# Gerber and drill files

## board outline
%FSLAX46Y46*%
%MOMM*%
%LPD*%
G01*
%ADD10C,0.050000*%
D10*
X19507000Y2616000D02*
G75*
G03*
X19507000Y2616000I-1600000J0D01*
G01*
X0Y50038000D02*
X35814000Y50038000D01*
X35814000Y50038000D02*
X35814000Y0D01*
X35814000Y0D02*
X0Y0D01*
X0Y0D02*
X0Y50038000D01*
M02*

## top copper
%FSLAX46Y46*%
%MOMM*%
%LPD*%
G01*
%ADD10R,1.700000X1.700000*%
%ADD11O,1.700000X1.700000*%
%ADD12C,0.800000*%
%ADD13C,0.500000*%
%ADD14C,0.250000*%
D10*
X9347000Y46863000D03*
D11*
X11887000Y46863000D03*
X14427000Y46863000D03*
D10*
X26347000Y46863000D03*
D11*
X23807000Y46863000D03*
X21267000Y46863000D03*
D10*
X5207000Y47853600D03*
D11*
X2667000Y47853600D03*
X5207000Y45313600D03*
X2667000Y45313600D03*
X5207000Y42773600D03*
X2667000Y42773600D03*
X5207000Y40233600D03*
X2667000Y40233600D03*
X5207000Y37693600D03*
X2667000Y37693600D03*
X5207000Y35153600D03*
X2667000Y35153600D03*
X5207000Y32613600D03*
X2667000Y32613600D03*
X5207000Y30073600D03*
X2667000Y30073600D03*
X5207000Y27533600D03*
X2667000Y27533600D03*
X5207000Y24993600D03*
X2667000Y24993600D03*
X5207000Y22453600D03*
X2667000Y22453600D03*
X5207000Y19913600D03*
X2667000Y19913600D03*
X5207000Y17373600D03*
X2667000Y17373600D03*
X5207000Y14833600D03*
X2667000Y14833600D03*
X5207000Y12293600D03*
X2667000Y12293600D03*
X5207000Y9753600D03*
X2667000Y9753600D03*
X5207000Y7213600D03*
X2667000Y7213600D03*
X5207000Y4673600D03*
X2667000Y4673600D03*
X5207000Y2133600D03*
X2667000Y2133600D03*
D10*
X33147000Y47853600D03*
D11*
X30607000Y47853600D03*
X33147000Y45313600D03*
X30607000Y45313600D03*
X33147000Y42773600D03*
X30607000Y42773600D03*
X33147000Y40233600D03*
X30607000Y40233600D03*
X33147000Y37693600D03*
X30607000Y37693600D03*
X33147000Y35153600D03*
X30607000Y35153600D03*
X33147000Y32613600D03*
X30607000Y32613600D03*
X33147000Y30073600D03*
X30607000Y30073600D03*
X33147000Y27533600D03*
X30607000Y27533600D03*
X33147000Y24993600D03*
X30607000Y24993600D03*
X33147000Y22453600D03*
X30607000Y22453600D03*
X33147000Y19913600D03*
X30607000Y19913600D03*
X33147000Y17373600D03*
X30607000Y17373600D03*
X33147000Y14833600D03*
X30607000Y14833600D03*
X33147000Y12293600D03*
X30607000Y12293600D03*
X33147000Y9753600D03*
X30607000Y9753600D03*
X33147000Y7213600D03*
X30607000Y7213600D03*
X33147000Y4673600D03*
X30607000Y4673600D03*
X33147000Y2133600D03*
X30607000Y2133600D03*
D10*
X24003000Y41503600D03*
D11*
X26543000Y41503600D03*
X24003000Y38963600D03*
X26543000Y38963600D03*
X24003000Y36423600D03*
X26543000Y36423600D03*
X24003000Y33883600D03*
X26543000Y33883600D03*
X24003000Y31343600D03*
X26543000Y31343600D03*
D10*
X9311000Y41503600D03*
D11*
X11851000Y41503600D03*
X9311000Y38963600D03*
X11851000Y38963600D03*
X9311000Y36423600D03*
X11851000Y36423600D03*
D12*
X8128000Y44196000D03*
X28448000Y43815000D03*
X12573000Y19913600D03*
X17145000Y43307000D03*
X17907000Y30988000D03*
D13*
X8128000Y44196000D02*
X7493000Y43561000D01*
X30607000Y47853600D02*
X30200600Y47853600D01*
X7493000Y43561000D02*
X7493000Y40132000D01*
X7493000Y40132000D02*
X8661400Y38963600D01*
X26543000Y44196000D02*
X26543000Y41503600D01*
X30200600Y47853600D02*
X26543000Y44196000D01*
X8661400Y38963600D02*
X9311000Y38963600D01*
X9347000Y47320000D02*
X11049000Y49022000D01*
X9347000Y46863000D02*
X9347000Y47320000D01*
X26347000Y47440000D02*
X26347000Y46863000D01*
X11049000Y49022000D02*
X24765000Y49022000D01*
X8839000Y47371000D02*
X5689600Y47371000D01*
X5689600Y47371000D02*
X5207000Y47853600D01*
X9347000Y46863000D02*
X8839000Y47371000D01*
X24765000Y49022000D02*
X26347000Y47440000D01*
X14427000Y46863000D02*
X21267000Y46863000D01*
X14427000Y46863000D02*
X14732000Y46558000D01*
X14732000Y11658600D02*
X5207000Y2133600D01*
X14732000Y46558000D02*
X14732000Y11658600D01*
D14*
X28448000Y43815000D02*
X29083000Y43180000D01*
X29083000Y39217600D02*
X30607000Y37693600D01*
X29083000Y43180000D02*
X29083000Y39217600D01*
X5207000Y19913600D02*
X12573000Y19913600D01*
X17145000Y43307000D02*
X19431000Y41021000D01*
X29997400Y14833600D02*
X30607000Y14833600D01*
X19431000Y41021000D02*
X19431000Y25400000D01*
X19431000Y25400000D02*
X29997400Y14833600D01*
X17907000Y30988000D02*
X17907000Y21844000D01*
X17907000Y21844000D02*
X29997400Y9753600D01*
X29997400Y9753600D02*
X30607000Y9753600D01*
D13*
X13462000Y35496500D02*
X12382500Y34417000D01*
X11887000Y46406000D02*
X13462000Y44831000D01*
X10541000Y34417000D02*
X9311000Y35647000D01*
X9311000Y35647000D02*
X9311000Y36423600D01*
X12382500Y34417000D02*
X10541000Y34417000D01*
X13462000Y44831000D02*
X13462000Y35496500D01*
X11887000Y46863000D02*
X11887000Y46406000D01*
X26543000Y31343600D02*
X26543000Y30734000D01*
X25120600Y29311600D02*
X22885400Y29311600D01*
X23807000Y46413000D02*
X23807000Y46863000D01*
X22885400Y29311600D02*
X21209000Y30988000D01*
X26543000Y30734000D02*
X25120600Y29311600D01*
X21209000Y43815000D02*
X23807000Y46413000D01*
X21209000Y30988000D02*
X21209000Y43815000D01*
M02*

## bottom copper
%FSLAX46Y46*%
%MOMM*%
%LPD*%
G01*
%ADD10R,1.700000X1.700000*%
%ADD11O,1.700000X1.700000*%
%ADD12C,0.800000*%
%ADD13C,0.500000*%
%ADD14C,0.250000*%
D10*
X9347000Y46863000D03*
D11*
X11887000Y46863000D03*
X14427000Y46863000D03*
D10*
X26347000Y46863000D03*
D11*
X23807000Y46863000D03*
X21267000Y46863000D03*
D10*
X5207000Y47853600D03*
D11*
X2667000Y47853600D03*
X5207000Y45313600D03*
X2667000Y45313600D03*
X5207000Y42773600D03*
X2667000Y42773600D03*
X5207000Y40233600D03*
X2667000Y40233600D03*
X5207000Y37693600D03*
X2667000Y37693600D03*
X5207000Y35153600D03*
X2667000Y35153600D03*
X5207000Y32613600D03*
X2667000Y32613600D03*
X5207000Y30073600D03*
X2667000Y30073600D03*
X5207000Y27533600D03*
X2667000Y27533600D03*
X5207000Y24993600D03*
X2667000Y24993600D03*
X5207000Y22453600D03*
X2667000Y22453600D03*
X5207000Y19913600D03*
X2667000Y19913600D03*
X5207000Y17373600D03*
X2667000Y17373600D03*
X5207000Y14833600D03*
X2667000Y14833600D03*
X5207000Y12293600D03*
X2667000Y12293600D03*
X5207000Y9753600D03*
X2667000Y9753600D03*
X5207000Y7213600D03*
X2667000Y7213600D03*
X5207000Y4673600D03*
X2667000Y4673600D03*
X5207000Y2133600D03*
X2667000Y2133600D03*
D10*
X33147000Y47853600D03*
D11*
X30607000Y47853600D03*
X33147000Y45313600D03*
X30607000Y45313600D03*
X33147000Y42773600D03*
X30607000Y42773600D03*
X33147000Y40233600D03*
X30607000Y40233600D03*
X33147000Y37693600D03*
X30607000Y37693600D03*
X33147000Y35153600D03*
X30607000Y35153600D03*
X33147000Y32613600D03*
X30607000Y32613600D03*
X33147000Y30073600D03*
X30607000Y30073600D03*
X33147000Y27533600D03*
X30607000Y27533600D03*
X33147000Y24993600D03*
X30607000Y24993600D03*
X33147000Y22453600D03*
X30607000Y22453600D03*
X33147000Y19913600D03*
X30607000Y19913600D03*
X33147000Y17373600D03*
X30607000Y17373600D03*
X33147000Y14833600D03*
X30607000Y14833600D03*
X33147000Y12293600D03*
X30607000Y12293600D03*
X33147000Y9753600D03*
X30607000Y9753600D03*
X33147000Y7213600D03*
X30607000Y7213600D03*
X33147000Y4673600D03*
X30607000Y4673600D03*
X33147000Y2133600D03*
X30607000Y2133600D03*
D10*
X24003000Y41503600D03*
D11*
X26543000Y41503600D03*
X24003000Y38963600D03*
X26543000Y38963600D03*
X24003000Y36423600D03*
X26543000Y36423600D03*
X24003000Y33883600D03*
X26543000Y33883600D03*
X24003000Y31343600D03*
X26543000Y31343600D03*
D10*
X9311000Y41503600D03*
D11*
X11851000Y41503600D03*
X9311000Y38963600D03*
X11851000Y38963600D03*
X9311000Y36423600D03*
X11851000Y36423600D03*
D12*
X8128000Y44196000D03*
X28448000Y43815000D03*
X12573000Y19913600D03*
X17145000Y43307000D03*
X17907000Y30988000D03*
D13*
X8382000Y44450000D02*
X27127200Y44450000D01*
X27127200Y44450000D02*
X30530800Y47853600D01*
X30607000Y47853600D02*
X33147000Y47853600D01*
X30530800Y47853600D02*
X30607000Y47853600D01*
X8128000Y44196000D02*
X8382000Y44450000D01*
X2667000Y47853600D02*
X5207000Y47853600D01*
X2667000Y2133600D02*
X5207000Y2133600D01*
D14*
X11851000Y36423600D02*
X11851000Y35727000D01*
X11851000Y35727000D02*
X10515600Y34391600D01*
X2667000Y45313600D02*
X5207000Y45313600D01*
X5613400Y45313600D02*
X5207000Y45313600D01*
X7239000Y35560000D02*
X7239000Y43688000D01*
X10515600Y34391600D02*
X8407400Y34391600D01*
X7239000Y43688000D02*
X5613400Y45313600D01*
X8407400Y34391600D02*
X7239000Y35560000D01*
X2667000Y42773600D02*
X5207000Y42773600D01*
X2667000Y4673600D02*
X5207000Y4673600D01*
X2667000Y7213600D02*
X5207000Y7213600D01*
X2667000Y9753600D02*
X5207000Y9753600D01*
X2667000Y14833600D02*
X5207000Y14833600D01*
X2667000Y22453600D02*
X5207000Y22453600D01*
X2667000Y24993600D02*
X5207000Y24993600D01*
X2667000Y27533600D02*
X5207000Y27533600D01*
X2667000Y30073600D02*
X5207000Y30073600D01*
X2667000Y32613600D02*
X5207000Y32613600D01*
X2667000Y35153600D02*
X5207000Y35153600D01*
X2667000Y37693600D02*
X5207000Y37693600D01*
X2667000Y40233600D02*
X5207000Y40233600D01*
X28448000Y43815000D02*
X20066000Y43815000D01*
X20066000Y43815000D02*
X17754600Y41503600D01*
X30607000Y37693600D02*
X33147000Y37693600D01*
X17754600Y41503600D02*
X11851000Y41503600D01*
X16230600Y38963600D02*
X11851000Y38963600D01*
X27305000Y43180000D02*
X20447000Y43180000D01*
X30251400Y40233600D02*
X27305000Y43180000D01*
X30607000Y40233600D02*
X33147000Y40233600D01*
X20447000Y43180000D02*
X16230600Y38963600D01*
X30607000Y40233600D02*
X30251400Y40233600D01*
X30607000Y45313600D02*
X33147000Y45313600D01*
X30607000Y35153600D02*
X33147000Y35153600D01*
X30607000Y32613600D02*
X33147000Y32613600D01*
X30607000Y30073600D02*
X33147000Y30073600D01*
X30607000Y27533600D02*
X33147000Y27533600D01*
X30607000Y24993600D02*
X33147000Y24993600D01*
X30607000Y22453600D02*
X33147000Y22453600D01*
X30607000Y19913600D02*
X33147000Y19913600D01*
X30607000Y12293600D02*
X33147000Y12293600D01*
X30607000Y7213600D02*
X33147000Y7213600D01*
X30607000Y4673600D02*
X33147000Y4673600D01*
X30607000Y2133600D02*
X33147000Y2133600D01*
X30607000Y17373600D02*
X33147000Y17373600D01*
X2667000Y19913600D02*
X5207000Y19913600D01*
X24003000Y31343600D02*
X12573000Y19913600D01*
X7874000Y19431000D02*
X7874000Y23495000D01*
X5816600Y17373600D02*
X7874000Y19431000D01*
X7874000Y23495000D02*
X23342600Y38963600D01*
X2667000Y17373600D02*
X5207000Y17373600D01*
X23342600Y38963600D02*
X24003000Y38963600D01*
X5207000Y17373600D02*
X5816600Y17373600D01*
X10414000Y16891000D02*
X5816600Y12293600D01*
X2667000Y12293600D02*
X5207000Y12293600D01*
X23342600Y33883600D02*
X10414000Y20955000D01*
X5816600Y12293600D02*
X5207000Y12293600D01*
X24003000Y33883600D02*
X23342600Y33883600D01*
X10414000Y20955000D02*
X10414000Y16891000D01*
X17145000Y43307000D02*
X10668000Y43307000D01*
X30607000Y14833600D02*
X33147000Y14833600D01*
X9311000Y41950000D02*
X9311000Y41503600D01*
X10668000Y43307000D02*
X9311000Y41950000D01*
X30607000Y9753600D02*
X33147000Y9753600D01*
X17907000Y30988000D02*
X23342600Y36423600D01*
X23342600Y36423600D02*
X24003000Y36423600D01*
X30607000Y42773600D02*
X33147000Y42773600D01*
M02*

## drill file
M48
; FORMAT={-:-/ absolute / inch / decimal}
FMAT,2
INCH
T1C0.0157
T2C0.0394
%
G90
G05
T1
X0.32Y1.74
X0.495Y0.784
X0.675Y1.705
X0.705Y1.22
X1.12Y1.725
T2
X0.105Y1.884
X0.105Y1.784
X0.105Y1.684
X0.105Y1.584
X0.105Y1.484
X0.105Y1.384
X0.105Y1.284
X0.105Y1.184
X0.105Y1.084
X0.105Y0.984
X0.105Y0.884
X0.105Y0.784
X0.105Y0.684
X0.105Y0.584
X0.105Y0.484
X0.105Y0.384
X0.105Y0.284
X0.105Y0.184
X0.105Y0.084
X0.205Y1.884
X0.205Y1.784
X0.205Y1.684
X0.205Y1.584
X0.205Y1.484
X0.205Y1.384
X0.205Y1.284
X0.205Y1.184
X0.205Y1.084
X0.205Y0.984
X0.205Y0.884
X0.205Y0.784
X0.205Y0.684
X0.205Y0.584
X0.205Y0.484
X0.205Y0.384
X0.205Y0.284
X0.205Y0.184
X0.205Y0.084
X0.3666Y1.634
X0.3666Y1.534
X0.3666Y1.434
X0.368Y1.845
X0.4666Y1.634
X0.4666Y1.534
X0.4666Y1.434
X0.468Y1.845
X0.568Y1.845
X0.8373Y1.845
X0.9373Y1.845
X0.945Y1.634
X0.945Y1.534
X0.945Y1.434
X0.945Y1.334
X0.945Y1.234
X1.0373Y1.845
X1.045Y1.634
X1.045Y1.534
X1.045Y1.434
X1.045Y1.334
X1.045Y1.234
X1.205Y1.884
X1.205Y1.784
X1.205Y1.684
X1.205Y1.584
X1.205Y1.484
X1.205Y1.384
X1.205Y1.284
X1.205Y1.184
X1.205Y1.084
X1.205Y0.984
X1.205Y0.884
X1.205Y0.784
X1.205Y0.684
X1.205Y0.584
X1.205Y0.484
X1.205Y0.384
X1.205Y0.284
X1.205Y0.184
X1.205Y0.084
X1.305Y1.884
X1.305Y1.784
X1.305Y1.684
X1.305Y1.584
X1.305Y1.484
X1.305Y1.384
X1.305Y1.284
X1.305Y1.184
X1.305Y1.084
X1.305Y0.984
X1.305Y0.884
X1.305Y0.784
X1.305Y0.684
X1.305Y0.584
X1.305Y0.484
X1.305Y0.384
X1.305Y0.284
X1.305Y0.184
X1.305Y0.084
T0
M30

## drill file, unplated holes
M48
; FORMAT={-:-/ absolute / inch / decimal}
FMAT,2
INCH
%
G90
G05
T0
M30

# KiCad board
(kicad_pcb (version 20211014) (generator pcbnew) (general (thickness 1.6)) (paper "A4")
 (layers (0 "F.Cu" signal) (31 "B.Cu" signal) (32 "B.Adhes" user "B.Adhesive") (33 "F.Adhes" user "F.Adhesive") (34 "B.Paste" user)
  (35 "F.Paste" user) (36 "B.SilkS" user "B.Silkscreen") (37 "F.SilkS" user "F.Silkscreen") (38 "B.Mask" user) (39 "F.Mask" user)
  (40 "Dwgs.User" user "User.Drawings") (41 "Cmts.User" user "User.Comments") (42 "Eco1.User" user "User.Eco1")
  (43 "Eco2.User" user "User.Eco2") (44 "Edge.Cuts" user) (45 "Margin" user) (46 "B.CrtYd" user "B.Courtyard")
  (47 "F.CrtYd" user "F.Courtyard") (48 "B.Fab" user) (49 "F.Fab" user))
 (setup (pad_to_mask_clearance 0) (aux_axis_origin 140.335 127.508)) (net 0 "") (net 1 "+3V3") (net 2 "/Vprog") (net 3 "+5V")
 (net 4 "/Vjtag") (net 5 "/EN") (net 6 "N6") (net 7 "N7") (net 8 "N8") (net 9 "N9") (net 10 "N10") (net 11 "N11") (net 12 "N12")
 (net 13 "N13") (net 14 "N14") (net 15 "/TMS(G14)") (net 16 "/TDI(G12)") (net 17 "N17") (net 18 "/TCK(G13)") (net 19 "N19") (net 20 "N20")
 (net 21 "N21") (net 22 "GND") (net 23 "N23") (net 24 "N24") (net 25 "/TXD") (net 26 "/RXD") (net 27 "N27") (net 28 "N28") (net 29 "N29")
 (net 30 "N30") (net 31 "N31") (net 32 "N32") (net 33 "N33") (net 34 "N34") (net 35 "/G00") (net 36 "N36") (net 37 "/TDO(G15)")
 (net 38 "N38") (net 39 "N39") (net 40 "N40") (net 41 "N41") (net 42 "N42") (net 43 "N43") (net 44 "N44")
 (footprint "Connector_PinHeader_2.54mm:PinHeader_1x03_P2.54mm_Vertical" (layer "F.Cu") (at 149.682 80.645 90)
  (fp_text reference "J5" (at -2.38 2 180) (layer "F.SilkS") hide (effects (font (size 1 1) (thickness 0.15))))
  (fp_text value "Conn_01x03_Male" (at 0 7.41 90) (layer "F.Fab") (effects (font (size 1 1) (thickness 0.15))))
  (pad "1" thru_hole rect locked (at 0 0 90) (size 1.7 1.7) (drill 1) (layers *.Cu *.Mask) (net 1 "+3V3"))
  (pad "2" thru_hole oval locked (at 0 2.54 90) (size 1.7 1.7) (drill 1) (layers *.Cu *.Mask) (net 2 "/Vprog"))
  (pad "3" thru_hole oval locked (at 0 5.08 90) (size 1.7 1.7) (drill 1) (layers *.Cu *.Mask) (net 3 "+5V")))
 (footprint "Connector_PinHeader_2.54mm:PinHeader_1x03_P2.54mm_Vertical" (layer "F.Cu") (at 166.682 80.645 -90)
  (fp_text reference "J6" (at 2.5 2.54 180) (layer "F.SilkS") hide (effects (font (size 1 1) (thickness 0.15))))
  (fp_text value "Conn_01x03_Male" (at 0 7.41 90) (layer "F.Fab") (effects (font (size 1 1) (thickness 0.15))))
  (pad "1" thru_hole rect locked (at 0 0 270) (size 1.7 1.7) (drill 1) (layers *.Cu *.Mask) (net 1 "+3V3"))
  (pad "2" thru_hole oval locked (at 0 2.54 270) (size 1.7 1.7) (drill 1) (layers *.Cu *.Mask) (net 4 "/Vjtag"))
  (pad "3" thru_hole oval locked (at 0 5.08 270) (size 1.7 1.7) (drill 1) (layers *.Cu *.Mask) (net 3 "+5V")))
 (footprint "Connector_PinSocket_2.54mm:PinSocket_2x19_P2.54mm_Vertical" (layer "F.Cu") (at 145.542 79.6544)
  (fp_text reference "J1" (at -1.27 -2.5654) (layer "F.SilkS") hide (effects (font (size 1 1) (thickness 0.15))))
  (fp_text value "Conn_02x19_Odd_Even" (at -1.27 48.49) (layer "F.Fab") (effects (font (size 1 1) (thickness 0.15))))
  (pad "1" thru_hole rect locked (at 0 0) (size 1.7 1.7) (drill 1) (layers *.Cu *.Mask) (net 1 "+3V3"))
  (pad "2" thru_hole oval locked (at -2.54 0) (size 1.7 1.7) (drill 1) (layers *.Cu *.Mask) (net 1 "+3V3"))
  (pad "3" thru_hole oval locked (at 0 2.54) (size 1.7 1.7) (drill 1) (layers *.Cu *.Mask) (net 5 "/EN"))
  (pad "4" thru_hole oval locked (at -2.54 2.54) (size 1.7 1.7) (drill 1) (layers *.Cu *.Mask) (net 5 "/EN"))
  (pad "5" thru_hole oval locked (at 0 5.08) (size 1.7 1.7) (drill 1) (layers *.Cu *.Mask) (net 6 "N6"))
  (pad "6" thru_hole oval locked (at -2.54 5.08) (size 1.7 1.7) (drill 1) (layers *.Cu *.Mask) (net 6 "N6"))
  (pad "7" thru_hole oval locked (at 0 7.62) (size 1.7 1.7) (drill 1) (layers *.Cu *.Mask) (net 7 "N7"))
  (pad "8" thru_hole oval locked (at -2.54 7.62) (size 1.7 1.7) (drill 1) (layers *.Cu *.Mask) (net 7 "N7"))
  (pad "9" thru_hole oval locked (at 0 10.16) (size 1.7 1.7) (drill 1) (layers *.Cu *.Mask) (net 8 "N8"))
  (pad "10" thru_hole oval locked (at -2.54 10.16) (size 1.7 1.7) (drill 1) (layers *.Cu *.Mask) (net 8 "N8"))
  (pad "11" thru_hole oval locked (at 0 12.7) (size 1.7 1.7) (drill 1) (layers *.Cu *.Mask) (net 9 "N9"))
  (pad "12" thru_hole oval locked (at -2.54 12.7) (size 1.7 1.7) (drill 1) (layers *.Cu *.Mask) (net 9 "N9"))
  (pad "13" thru_hole oval locked (at 0 15.24) (size 1.7 1.7) (drill 1) (layers *.Cu *.Mask) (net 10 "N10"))
  (pad "14" thru_hole oval locked (at -2.54 15.24) (size 1.7 1.7) (drill 1) (layers *.Cu *.Mask) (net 10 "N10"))
  (pad "15" thru_hole oval locked (at 0 17.78) (size 1.7 1.7) (drill 1) (layers *.Cu *.Mask) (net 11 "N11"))
  (pad "16" thru_hole oval locked (at -2.54 17.78) (size 1.7 1.7) (drill 1) (layers *.Cu *.Mask) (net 11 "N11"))
  (pad "17" thru_hole oval locked (at 0 20.32) (size 1.7 1.7) (drill 1) (layers *.Cu *.Mask) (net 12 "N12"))
  (pad "18" thru_hole oval locked (at -2.54 20.32) (size 1.7 1.7) (drill 1) (layers *.Cu *.Mask) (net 12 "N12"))
  (pad "19" thru_hole oval locked (at 0 22.86) (size 1.7 1.7) (drill 1) (layers *.Cu *.Mask) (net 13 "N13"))
  (pad "20" thru_hole oval locked (at -2.54 22.86) (size 1.7 1.7) (drill 1) (layers *.Cu *.Mask) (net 13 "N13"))
  (pad "21" thru_hole oval locked (at 0 25.4) (size 1.7 1.7) (drill 1) (layers *.Cu *.Mask) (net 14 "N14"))
  (pad "22" thru_hole oval locked (at -2.54 25.4) (size 1.7 1.7) (drill 1) (layers *.Cu *.Mask) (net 14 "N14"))
  (pad "23" thru_hole oval locked (at 0 27.94) (size 1.7 1.7) (drill 1) (layers *.Cu *.Mask) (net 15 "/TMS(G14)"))
  (pad "24" thru_hole oval locked (at -2.54 27.94) (size 1.7 1.7) (drill 1) (layers *.Cu *.Mask) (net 15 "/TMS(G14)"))
  (pad "25" thru_hole oval locked (at 0 30.48) (size 1.7 1.7) (drill 1) (layers *.Cu *.Mask) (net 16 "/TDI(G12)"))
  (pad "26" thru_hole oval locked (at -2.54 30.48) (size 1.7 1.7) (drill 1) (layers *.Cu *.Mask) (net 16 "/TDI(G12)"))
  (pad "27" thru_hole oval locked (at 0 33.02) (size 1.7 1.7) (drill 1) (layers *.Cu *.Mask) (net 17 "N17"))
  (pad "28" thru_hole oval locked (at -2.54 33.02) (size 1.7 1.7) (drill 1) (layers *.Cu *.Mask) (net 17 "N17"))
  (pad "29" thru_hole oval locked (at 0 35.56) (size 1.7 1.7) (drill 1) (layers *.Cu *.Mask) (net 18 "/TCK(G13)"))
  (pad "30" thru_hole oval locked (at -2.54 35.56) (size 1.7 1.7) (drill 1) (layers *.Cu *.Mask) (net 18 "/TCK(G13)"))
  (pad "31" thru_hole oval locked (at 0 38.1) (size 1.7 1.7) (drill 1) (layers *.Cu *.Mask) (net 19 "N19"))
  (pad "32" thru_hole oval locked (at -2.54 38.1) (size 1.7 1.7) (drill 1) (layers *.Cu *.Mask) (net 19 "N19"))
  (pad "33" thru_hole oval locked (at 0 40.64) (size 1.7 1.7) (drill 1) (layers *.Cu *.Mask) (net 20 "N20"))
  (pad "34" thru_hole oval locked (at -2.54 40.64) (size 1.7 1.7) (drill 1) (layers *.Cu *.Mask) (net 20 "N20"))
  (pad "35" thru_hole oval locked (at 0 43.18) (size 1.7 1.7) (drill 1) (layers *.Cu *.Mask) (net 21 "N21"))
  (pad "36" thru_hole oval locked (at -2.54 43.18) (size 1.7 1.7) (drill 1) (layers *.Cu *.Mask) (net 21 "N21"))
  (pad "37" thru_hole oval locked (at 0 45.72) (size 1.7 1.7) (drill 1) (layers *.Cu *.Mask) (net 3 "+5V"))
  (pad "38" thru_hole oval locked (at -2.54 45.72) (size 1.7 1.7) (drill 1) (layers *.Cu *.Mask) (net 3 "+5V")))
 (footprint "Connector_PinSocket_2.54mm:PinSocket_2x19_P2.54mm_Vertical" (layer "F.Cu") (at 173.482 79.6544)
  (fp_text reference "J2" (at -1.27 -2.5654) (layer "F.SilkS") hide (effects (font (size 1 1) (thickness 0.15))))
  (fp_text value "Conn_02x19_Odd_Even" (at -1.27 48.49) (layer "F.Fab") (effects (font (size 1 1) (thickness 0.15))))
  (pad "1" thru_hole rect locked (at 0 0) (size 1.7 1.7) (drill 1) (layers *.Cu *.Mask) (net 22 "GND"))
  (pad "2" thru_hole oval locked (at -2.54 0) (size 1.7 1.7) (drill 1) (layers *.Cu *.Mask) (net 22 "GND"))
  (pad "3" thru_hole oval locked (at 0 2.54) (size 1.7 1.7) (drill 1) (layers *.Cu *.Mask) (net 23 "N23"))
  (pad "4" thru_hole oval locked (at -2.54 2.54) (size 1.7 1.7) (drill 1) (layers *.Cu *.Mask) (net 23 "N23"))
  (pad "5" thru_hole oval locked (at 0 5.08) (size 1.7 1.7) (drill 1) (layers *.Cu *.Mask) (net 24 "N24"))
  (pad "6" thru_hole oval locked (at -2.54 5.08) (size 1.7 1.7) (drill 1) (layers *.Cu *.Mask) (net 24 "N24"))
  (pad "7" thru_hole oval locked (at 0 7.62) (size 1.7 1.7) (drill 1) (layers *.Cu *.Mask) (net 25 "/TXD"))
  (pad "8" thru_hole oval locked (at -2.54 7.62) (size 1.7 1.7) (drill 1) (layers *.Cu *.Mask) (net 25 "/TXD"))
  (pad "9" thru_hole oval locked (at 0 10.16) (size 1.7 1.7) (drill 1) (layers *.Cu *.Mask) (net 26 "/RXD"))
  (pad "10" thru_hole oval locked (at -2.54 10.16) (size 1.7 1.7) (drill 1) (layers *.Cu *.Mask) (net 26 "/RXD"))
  (pad "11" thru_hole oval locked (at 0 12.7) (size 1.7 1.7) (drill 1) (layers *.Cu *.Mask) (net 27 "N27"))
  (pad "12" thru_hole oval locked (at -2.54 12.7) (size 1.7 1.7) (drill 1) (layers *.Cu *.Mask) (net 27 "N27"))
  (pad "13" thru_hole oval locked (at 0 15.24) (size 1.7 1.7) (drill 1) (layers *.Cu *.Mask) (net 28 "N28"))
  (pad "14" thru_hole oval locked (at -2.54 15.24) (size 1.7 1.7) (drill 1) (layers *.Cu *.Mask) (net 28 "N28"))
  (pad "15" thru_hole oval locked (at 0 17.78) (size 1.7 1.7) (drill 1) (layers *.Cu *.Mask) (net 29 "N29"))
  (pad "16" thru_hole oval locked (at -2.54 17.78) (size 1.7 1.7) (drill 1) (layers *.Cu *.Mask) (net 29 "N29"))
  (pad "17" thru_hole oval locked (at 0 20.32) (size 1.7 1.7) (drill 1) (layers *.Cu *.Mask) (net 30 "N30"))
  (pad "18" thru_hole oval locked (at -2.54 20.32) (size 1.7 1.7) (drill 1) (layers *.Cu *.Mask) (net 30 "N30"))
  (pad "19" thru_hole oval locked (at 0 22.86) (size 1.7 1.7) (drill 1) (layers *.Cu *.Mask) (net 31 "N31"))
  (pad "20" thru_hole oval locked (at -2.54 22.86) (size 1.7 1.7) (drill 1) (layers *.Cu *.Mask) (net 31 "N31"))
  (pad "21" thru_hole oval locked (at 0 25.4) (size 1.7 1.7) (drill 1) (layers *.Cu *.Mask) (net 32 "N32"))
  (pad "22" thru_hole oval locked (at -2.54 25.4) (size 1.7 1.7) (drill 1) (layers *.Cu *.Mask) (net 32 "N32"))
  (pad "23" thru_hole oval locked (at 0 27.94) (size 1.7 1.7) (drill 1) (layers *.Cu *.Mask) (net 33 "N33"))
  (pad "24" thru_hole oval locked (at -2.54 27.94) (size 1.7 1.7) (drill 1) (layers *.Cu *.Mask) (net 33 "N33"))
  (pad "25" thru_hole oval locked (at 0 30.48) (size 1.7 1.7) (drill 1) (layers *.Cu *.Mask) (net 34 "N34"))
  (pad "26" thru_hole oval locked (at -2.54 30.48) (size 1.7 1.7) (drill 1) (layers *.Cu *.Mask) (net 34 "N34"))
  (pad "27" thru_hole oval locked (at 0 33.02) (size 1.7 1.7) (drill 1) (layers *.Cu *.Mask) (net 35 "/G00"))
  (pad "28" thru_hole oval locked (at -2.54 33.02) (size 1.7 1.7) (drill 1) (layers *.Cu *.Mask) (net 35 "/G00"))
  (pad "29" thru_hole oval locked (at 0 35.56) (size 1.7 1.7) (drill 1) (layers *.Cu *.Mask) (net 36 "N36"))
  (pad "30" thru_hole oval locked (at -2.54 35.56) (size 1.7 1.7) (drill 1) (layers *.Cu *.Mask) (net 36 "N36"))
  (pad "31" thru_hole oval locked (at 0 38.1) (size 1.7 1.7) (drill 1) (layers *.Cu *.Mask) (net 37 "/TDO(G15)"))
  (pad "32" thru_hole oval locked (at -2.54 38.1) (size 1.7 1.7) (drill 1) (layers *.Cu *.Mask) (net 37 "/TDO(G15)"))
  (pad "33" thru_hole oval locked (at 0 40.64) (size 1.7 1.7) (drill 1) (layers *.Cu *.Mask) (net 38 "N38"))
  (pad "34" thru_hole oval locked (at -2.54 40.64) (size 1.7 1.7) (drill 1) (layers *.Cu *.Mask) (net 38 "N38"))
  (pad "35" thru_hole oval locked (at 0 43.18) (size 1.7 1.7) (drill 1) (layers *.Cu *.Mask) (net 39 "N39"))
  (pad "36" thru_hole oval locked (at -2.54 43.18) (size 1.7 1.7) (drill 1) (layers *.Cu *.Mask) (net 39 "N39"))
  (pad "37" thru_hole oval locked (at 0 45.72) (size 1.7 1.7) (drill 1) (layers *.Cu *.Mask) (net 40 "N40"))
  (pad "38" thru_hole oval locked (at -2.54 45.72) (size 1.7 1.7) (drill 1) (layers *.Cu *.Mask) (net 40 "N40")))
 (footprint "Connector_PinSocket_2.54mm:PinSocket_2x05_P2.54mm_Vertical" (layer "B.Cu") (at 164.338 86.0044 180)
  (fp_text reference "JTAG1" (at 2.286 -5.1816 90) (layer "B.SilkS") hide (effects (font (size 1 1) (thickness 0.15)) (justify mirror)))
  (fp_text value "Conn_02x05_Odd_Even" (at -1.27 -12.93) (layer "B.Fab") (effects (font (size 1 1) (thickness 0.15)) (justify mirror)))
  (pad "1" thru_hole rect locked (at 0 0 180) (size 1.7 1.7) (drill 1) (layers *.Cu *.Mask) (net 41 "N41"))
  (pad "2" thru_hole oval locked (at -2.54 0 180) (size 1.7 1.7) (drill 1) (layers *.Cu *.Mask) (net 22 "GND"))
  (pad "3" thru_hole oval locked (at 0 -2.54 180) (size 1.7 1.7) (drill 1) (layers *.Cu *.Mask) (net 16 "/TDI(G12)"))
  (pad "4" thru_hole oval locked (at -2.54 -2.54 180) (size 1.7 1.7) (drill 1) (layers *.Cu *.Mask) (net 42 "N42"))
  (pad "5" thru_hole oval locked (at 0 -5.08 180) (size 1.7 1.7) (drill 1) (layers *.Cu *.Mask) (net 37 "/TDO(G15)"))
  (pad "6" thru_hole oval locked (at -2.54 -5.08 180) (size 1.7 1.7) (drill 1) (layers *.Cu *.Mask) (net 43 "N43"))
  (pad "7" thru_hole oval locked (at 0 -7.62 180) (size 1.7 1.7) (drill 1) (layers *.Cu *.Mask) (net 18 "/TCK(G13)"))
  (pad "8" thru_hole oval locked (at -2.54 -7.62 180) (size 1.7 1.7) (drill 1) (layers *.Cu *.Mask) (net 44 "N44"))
  (pad "9" thru_hole oval locked (at 0 -10.16 180) (size 1.7 1.7) (drill 1) (layers *.Cu *.Mask) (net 15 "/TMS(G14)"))
  (pad "10" thru_hole oval locked (at -2.54 -10.16 180) (size 1.7 1.7) (drill 1) (layers *.Cu *.Mask) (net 4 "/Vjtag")))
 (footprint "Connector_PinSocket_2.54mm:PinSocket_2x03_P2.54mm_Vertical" (layer "B.Cu") (at 149.646 86.0044 180)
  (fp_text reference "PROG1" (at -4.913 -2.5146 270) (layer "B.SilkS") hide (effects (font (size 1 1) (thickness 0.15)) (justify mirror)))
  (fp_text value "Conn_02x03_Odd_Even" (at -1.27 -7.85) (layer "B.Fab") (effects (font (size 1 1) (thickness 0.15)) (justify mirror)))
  (pad "1" thru_hole rect locked (at 0 0 180) (size 1.7 1.7) (drill 1) (layers *.Cu *.Mask) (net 35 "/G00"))
  (pad "2" thru_hole oval locked (at -2.54 0 180) (size 1.7 1.7) (drill 1) (layers *.Cu *.Mask) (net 26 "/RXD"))
  (pad "3" thru_hole oval locked (at 0 -2.54 180) (size 1.7 1.7) (drill 1) (layers *.Cu *.Mask) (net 22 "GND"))
  (pad "4" thru_hole oval locked (at -2.54 -2.54 180) (size 1.7 1.7) (drill 1) (layers *.Cu *.Mask) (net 25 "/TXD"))
  (pad "5" thru_hole oval locked (at 0 -5.08 180) (size 1.7 1.7) (drill 1) (layers *.Cu *.Mask) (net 2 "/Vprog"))
  (pad "6" thru_hole oval locked (at -2.54 -5.08 180) (size 1.7 1.7) (drill 1) (layers *.Cu *.Mask) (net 5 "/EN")))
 (gr_circle (center 158.242 124.892) (end 159.842 124.892) (layer "Edge.Cuts") (width 0.05) (fill none))
 (gr_rect (start 140.335 77.47) (end 176.149 127.508) (layer "Edge.Cuts") (width 0.05) (fill none))
 (segment (start 148.463 83.312) (end 147.828 83.947) (width 0.5) (layer "F.Cu") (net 22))
 (segment (start 170.942 79.6544) (end 170.5356 79.6544) (width 0.5) (layer "F.Cu") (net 22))
 (segment (start 147.828 83.947) (end 147.828 87.376) (width 0.5) (layer "F.Cu") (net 22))
 (segment (start 147.828 87.376) (end 148.9964 88.5444) (width 0.5) (layer "F.Cu") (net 22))
 (segment (start 166.878 83.312) (end 166.878 86.0044) (width 0.5) (layer "F.Cu") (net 22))
 (segment (start 170.5356 79.6544) (end 166.878 83.312) (width 0.5) (layer "F.Cu") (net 22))
 (segment (start 148.9964 88.5444) (end 149.646 88.5444) (width 0.5) (layer "F.Cu") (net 22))
 (via (at 148.463 83.312) (size 0.8) (drill 0.4) (layers "F.Cu" "B.Cu") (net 22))
 (segment (start 148.717 83.058) (end 167.4622 83.058) (width 0.5) (layer "B.Cu") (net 22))
 (segment (start 167.4622 83.058) (end 170.8658 79.6544) (width 0.5) (layer "B.Cu") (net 22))
 (segment (start 170.942 79.6544) (end 173.482 79.6544) (width 0.5) (layer "B.Cu") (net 22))
 (segment (start 170.8658 79.6544) (end 170.942 79.6544) (width 0.5) (layer "B.Cu") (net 22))
 (segment (start 148.463 83.312) (end 148.717 83.058) (width 0.5) (layer "B.Cu") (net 22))
 (segment (start 149.682 80.188) (end 151.384 78.486) (width 0.5) (layer "F.Cu") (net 1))
 (segment (start 149.682 80.645) (end 149.682 80.188) (width 0.5) (layer "F.Cu") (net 1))
 (segment (start 166.682 80.068) (end 166.682 80.645) (width 0.5) (layer "F.Cu") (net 1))
 (segment (start 151.384 78.486) (end 165.1 78.486) (width 0.5) (layer "F.Cu") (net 1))
 (segment (start 149.174 80.137) (end 146.0246 80.137) (width 0.5) (layer "F.Cu") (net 1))
 (segment (start 146.0246 80.137) (end 145.542 79.6544) (width 0.5) (layer "F.Cu") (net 1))
 (segment (start 149.682 80.645) (end 149.174 80.137) (width 0.5) (layer "F.Cu") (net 1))
 (segment (start 165.1 78.486) (end 166.682 80.068) (width 0.5) (layer "F.Cu") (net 1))
 (segment (start 143.002 79.6544) (end 145.542 79.6544) (width 0.5) (layer "B.Cu") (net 1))
 (segment (start 154.762 80.645) (end 161.602 80.645) (width 0.5) (layer "F.Cu") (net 3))
 (segment (start 154.762 80.645) (end 155.067 80.95) (width 0.5) (layer "F.Cu") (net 3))
 (segment (start 155.067 115.8494) (end 145.542 125.3744) (width 0.5) (layer "F.Cu") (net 3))
 (segment (start 155.067 80.95) (end 155.067 115.8494) (width 0.5) (layer "F.Cu") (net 3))
 (segment (start 143.002 125.3744) (end 145.542 125.3744) (width 0.5) (layer "B.Cu") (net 3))
 (segment (start 152.186 91.0844) (end 152.186 91.781) (width 0.25) (layer "B.Cu") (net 5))
 (segment (start 152.186 91.781) (end 150.8506 93.1164) (width 0.25) (layer "B.Cu") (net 5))
 (segment (start 143.002 82.1944) (end 145.542 82.1944) (width 0.25) (layer "B.Cu") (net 5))
 (segment (start 145.9484 82.1944) (end 145.542 82.1944) (width 0.25) (layer "B.Cu") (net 5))
 (segment (start 147.574 91.948) (end 147.574 83.82) (width 0.25) (layer "B.Cu") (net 5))
 (segment (start 150.8506 93.1164) (end 148.7424 93.1164) (width 0.25) (layer "B.Cu") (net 5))
 (segment (start 147.574 83.82) (end 145.9484 82.1944) (width 0.25) (layer "B.Cu") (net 5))
 (segment (start 148.7424 93.1164) (end 147.574 91.948) (width 0.25) (layer "B.Cu") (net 5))
 (segment (start 143.002 84.7344) (end 145.542 84.7344) (width 0.25) (layer "B.Cu") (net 6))
 (segment (start 143.002 122.8344) (end 145.542 122.8344) (width 0.25) (layer "B.Cu") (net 21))
 (segment (start 143.002 120.2944) (end 145.542 120.2944) (width 0.25) (layer "B.Cu") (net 20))
 (segment (start 143.002 117.7544) (end 145.542 117.7544) (width 0.25) (layer "B.Cu") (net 19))
 (segment (start 143.002 112.6744) (end 145.542 112.6744) (width 0.25) (layer "B.Cu") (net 17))
 (segment (start 143.002 105.0544) (end 145.542 105.0544) (width 0.25) (layer "B.Cu") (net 14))
 (segment (start 143.002 102.5144) (end 145.542 102.5144) (width 0.25) (layer "B.Cu") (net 13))
 (segment (start 143.002 99.9744) (end 145.542 99.9744) (width 0.25) (layer "B.Cu") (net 12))
 (segment (start 143.002 97.4344) (end 145.542 97.4344) (width 0.25) (layer "B.Cu") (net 11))
 (segment (start 143.002 94.8944) (end 145.542 94.8944) (width 0.25) (layer "B.Cu") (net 10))
 (segment (start 143.002 92.3544) (end 145.542 92.3544) (width 0.25) (layer "B.Cu") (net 9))
 (segment (start 143.002 89.8144) (end 145.542 89.8144) (width 0.25) (layer "B.Cu") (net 8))
 (segment (start 143.002 87.2744) (end 145.542 87.2744) (width 0.25) (layer "B.Cu") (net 7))
 (segment (start 168.783 83.693) (end 169.418 84.328) (width 0.25) (layer "F.Cu") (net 26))
 (segment (start 169.418 88.2904) (end 170.942 89.8144) (width 0.25) (layer "F.Cu") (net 26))
 (segment (start 169.418 84.328) (end 169.418 88.2904) (width 0.25) (layer "F.Cu") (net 26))
 (via (at 168.783 83.693) (size 0.8) (drill 0.4) (layers "F.Cu" "B.Cu") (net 26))
 (segment (start 168.783 83.693) (end 160.401 83.693) (width 0.25) (layer "B.Cu") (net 26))
 (segment (start 160.401 83.693) (end 158.0896 86.0044) (width 0.25) (layer "B.Cu") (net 26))
 (segment (start 170.942 89.8144) (end 173.482 89.8144) (width 0.25) (layer "B.Cu") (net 26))
 (segment (start 158.0896 86.0044) (end 152.186 86.0044) (width 0.25) (layer "B.Cu") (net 26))
 (segment (start 156.5656 88.5444) (end 152.186 88.5444) (width 0.25) (layer "B.Cu") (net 25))
 (segment (start 167.64 84.328) (end 160.782 84.328) (width 0.25) (layer "B.Cu") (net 25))
 (segment (start 170.5864 87.2744) (end 167.64 84.328) (width 0.25) (layer "B.Cu") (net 25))
 (segment (start 170.942 87.2744) (end 173.482 87.2744) (width 0.25) (layer "B.Cu") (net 25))
 (segment (start 160.782 84.328) (end 156.5656 88.5444) (width 0.25) (layer "B.Cu") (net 25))
 (segment (start 170.942 87.2744) (end 170.5864 87.2744) (width 0.25) (layer "B.Cu") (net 25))
 (segment (start 170.942 82.1944) (end 173.482 82.1944) (width 0.25) (layer "B.Cu") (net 23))
 (segment (start 170.942 92.3544) (end 173.482 92.3544) (width 0.25) (layer "B.Cu") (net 27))
 (segment (start 170.942 94.8944) (end 173.482 94.8944) (width 0.25) (layer "B.Cu") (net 28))
 (segment (start 170.942 97.4344) (end 173.482 97.4344) (width 0.25) (layer "B.Cu") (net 29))
 (segment (start 170.942 99.9744) (end 173.482 99.9744) (width 0.25) (layer "B.Cu") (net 30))
 (segment (start 170.942 102.5144) (end 173.482 102.5144) (width 0.25) (layer "B.Cu") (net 31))
 (segment (start 170.942 105.0544) (end 173.482 105.0544) (width 0.25) (layer "B.Cu") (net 32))
 (segment (start 170.942 107.5944) (end 173.482 107.5944) (width 0.25) (layer "B.Cu") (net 33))
 (segment (start 170.942 115.2144) (end 173.482 115.2144) (width 0.25) (layer "B.Cu") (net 36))
 (segment (start 170.942 120.2944) (end 173.482 120.2944) (width 0.25) (layer "B.Cu") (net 38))
 (segment (start 170.942 122.8344) (end 173.482 122.8344) (width 0.25) (layer "B.Cu") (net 39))
 (segment (start 170.942 125.3744) (end 173.482 125.3744) (width 0.25) (layer "B.Cu") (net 40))
 (segment (start 170.942 110.1344) (end 173.482 110.1344) (width 0.25) (layer "B.Cu") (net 34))
 (segment (start 145.542 107.5944) (end 152.908 107.5944) (width 0.25) (layer "F.Cu") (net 15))
 (via (at 152.908 107.5944) (size 0.8) (drill 0.4) (layers "F.Cu" "B.Cu") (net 15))
 (segment (start 143.002 107.5944) (end 145.542 107.5944) (width 0.25) (layer "B.Cu") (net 15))
 (segment (start 164.338 96.1644) (end 152.908 107.5944) (width 0.25) (layer "B.Cu") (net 15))
 (segment (start 148.209 108.077) (end 148.209 104.013) (width 0.25) (layer "B.Cu") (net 16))
 (segment (start 146.1516 110.1344) (end 148.209 108.077) (width 0.25) (layer "B.Cu") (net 16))
 (segment (start 148.209 104.013) (end 163.6776 88.5444) (width 0.25) (layer "B.Cu") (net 16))
 (segment (start 143.002 110.1344) (end 145.542 110.1344) (width 0.25) (layer "B.Cu") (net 16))
 (segment (start 163.6776 88.5444) (end 164.338 88.5444) (width 0.25) (layer "B.Cu") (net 16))
 (segment (start 145.542 110.1344) (end 146.1516 110.1344) (width 0.25) (layer "B.Cu") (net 16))
 (segment (start 150.749 110.617) (end 146.1516 115.2144) (width 0.25) (layer "B.Cu") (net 18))
 (segment (start 143.002 115.2144) (end 145.542 115.2144) (width 0.25) (layer "B.Cu") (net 18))
 (segment (start 163.6776 93.6244) (end 150.749 106.553) (width 0.25) (layer "B.Cu") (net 18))
 (segment (start 146.1516 115.2144) (end 145.542 115.2144) (width 0.25) (layer "B.Cu") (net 18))
 (segment (start 164.338 93.6244) (end 163.6776 93.6244) (width 0.25) (layer "B.Cu") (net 18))
 (segment (start 150.749 106.553) (end 150.749 110.617) (width 0.25) (layer "B.Cu") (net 18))
 (segment (start 157.48 84.201) (end 159.766 86.487) (width 0.25) (layer "F.Cu") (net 35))
 (segment (start 170.3324 112.6744) (end 170.942 112.6744) (width 0.25) (layer "F.Cu") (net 35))
 (segment (start 159.766 86.487) (end 159.766 102.108) (width 0.25) (layer "F.Cu") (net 35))
 (segment (start 159.766 102.108) (end 170.3324 112.6744) (width 0.25) (layer "F.Cu") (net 35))
 (via (at 157.48 84.201) (size 0.8) (drill 0.4) (layers "F.Cu" "B.Cu") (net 35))
 (segment (start 157.48 84.201) (end 151.003 84.201) (width 0.25) (layer "B.Cu") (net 35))
 (segment (start 170.942 112.6744) (end 173.482 112.6744) (width 0.25) (layer "B.Cu") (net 35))
 (segment (start 149.646 85.558) (end 149.646 86.0044) (width 0.25) (layer "B.Cu") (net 35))
 (segment (start 151.003 84.201) (end 149.646 85.558) (width 0.25) (layer "B.Cu") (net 35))
 (segment (start 158.242 96.52) (end 158.242 105.664) (width 0.25) (layer "F.Cu") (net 37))
 (segment (start 158.242 105.664) (end 170.3324 117.7544) (width 0.25) (layer "F.Cu") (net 37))
 (segment (start 170.3324 117.7544) (end 170.942 117.7544) (width 0.25) (layer "F.Cu") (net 37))
 (via (at 158.242 96.52) (size 0.8) (drill 0.4) (layers "F.Cu" "B.Cu") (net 37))
 (segment (start 170.942 117.7544) (end 173.482 117.7544) (width 0.25) (layer "B.Cu") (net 37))
 (segment (start 158.242 96.52) (end 163.6776 91.0844) (width 0.25) (layer "B.Cu") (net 37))
 (segment (start 163.6776 91.0844) (end 164.338 91.0844) (width 0.25) (layer "B.Cu") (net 37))
 (segment (start 153.797 92.0115) (end 152.7175 93.091) (width 0.5) (layer "F.Cu") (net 2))
 (segment (start 152.222 81.102) (end 153.797 82.677) (width 0.5) (layer "F.Cu") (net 2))
 (segment (start 150.876 93.091) (end 149.646 91.861) (width 0.5) (layer "F.Cu") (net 2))
 (segment (start 149.646 91.861) (end 149.646 91.0844) (width 0.5) (layer "F.Cu") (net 2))
 (segment (start 152.7175 93.091) (end 150.876 93.091) (width 0.5) (layer "F.Cu") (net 2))
 (segment (start 153.797 82.677) (end 153.797 92.0115) (width 0.5) (layer "F.Cu") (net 2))
 (segment (start 152.222 80.645) (end 152.222 81.102) (width 0.5) (layer "F.Cu") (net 2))
 (segment (start 166.878 96.1644) (end 166.878 96.774) (width 0.5) (layer "F.Cu") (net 4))
 (segment (start 165.4556 98.1964) (end 163.2204 98.1964) (width 0.5) (layer "F.Cu") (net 4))
 (segment (start 164.142 81.095) (end 164.142 80.645) (width 0.5) (layer "F.Cu") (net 4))
 (segment (start 163.2204 98.1964) (end 161.544 96.52) (width 0.5) (layer "F.Cu") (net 4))
 (segment (start 166.878 96.774) (end 165.4556 98.1964) (width 0.5) (layer "F.Cu") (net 4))
 (segment (start 161.544 83.693) (end 164.142 81.095) (width 0.5) (layer "F.Cu") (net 4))
 (segment (start 161.544 96.52) (end 161.544 83.693) (width 0.5) (layer "F.Cu") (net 4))
 (segment (start 170.942 84.7344) (end 173.482 84.7344) (width 0.25) (layer "B.Cu") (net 24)))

